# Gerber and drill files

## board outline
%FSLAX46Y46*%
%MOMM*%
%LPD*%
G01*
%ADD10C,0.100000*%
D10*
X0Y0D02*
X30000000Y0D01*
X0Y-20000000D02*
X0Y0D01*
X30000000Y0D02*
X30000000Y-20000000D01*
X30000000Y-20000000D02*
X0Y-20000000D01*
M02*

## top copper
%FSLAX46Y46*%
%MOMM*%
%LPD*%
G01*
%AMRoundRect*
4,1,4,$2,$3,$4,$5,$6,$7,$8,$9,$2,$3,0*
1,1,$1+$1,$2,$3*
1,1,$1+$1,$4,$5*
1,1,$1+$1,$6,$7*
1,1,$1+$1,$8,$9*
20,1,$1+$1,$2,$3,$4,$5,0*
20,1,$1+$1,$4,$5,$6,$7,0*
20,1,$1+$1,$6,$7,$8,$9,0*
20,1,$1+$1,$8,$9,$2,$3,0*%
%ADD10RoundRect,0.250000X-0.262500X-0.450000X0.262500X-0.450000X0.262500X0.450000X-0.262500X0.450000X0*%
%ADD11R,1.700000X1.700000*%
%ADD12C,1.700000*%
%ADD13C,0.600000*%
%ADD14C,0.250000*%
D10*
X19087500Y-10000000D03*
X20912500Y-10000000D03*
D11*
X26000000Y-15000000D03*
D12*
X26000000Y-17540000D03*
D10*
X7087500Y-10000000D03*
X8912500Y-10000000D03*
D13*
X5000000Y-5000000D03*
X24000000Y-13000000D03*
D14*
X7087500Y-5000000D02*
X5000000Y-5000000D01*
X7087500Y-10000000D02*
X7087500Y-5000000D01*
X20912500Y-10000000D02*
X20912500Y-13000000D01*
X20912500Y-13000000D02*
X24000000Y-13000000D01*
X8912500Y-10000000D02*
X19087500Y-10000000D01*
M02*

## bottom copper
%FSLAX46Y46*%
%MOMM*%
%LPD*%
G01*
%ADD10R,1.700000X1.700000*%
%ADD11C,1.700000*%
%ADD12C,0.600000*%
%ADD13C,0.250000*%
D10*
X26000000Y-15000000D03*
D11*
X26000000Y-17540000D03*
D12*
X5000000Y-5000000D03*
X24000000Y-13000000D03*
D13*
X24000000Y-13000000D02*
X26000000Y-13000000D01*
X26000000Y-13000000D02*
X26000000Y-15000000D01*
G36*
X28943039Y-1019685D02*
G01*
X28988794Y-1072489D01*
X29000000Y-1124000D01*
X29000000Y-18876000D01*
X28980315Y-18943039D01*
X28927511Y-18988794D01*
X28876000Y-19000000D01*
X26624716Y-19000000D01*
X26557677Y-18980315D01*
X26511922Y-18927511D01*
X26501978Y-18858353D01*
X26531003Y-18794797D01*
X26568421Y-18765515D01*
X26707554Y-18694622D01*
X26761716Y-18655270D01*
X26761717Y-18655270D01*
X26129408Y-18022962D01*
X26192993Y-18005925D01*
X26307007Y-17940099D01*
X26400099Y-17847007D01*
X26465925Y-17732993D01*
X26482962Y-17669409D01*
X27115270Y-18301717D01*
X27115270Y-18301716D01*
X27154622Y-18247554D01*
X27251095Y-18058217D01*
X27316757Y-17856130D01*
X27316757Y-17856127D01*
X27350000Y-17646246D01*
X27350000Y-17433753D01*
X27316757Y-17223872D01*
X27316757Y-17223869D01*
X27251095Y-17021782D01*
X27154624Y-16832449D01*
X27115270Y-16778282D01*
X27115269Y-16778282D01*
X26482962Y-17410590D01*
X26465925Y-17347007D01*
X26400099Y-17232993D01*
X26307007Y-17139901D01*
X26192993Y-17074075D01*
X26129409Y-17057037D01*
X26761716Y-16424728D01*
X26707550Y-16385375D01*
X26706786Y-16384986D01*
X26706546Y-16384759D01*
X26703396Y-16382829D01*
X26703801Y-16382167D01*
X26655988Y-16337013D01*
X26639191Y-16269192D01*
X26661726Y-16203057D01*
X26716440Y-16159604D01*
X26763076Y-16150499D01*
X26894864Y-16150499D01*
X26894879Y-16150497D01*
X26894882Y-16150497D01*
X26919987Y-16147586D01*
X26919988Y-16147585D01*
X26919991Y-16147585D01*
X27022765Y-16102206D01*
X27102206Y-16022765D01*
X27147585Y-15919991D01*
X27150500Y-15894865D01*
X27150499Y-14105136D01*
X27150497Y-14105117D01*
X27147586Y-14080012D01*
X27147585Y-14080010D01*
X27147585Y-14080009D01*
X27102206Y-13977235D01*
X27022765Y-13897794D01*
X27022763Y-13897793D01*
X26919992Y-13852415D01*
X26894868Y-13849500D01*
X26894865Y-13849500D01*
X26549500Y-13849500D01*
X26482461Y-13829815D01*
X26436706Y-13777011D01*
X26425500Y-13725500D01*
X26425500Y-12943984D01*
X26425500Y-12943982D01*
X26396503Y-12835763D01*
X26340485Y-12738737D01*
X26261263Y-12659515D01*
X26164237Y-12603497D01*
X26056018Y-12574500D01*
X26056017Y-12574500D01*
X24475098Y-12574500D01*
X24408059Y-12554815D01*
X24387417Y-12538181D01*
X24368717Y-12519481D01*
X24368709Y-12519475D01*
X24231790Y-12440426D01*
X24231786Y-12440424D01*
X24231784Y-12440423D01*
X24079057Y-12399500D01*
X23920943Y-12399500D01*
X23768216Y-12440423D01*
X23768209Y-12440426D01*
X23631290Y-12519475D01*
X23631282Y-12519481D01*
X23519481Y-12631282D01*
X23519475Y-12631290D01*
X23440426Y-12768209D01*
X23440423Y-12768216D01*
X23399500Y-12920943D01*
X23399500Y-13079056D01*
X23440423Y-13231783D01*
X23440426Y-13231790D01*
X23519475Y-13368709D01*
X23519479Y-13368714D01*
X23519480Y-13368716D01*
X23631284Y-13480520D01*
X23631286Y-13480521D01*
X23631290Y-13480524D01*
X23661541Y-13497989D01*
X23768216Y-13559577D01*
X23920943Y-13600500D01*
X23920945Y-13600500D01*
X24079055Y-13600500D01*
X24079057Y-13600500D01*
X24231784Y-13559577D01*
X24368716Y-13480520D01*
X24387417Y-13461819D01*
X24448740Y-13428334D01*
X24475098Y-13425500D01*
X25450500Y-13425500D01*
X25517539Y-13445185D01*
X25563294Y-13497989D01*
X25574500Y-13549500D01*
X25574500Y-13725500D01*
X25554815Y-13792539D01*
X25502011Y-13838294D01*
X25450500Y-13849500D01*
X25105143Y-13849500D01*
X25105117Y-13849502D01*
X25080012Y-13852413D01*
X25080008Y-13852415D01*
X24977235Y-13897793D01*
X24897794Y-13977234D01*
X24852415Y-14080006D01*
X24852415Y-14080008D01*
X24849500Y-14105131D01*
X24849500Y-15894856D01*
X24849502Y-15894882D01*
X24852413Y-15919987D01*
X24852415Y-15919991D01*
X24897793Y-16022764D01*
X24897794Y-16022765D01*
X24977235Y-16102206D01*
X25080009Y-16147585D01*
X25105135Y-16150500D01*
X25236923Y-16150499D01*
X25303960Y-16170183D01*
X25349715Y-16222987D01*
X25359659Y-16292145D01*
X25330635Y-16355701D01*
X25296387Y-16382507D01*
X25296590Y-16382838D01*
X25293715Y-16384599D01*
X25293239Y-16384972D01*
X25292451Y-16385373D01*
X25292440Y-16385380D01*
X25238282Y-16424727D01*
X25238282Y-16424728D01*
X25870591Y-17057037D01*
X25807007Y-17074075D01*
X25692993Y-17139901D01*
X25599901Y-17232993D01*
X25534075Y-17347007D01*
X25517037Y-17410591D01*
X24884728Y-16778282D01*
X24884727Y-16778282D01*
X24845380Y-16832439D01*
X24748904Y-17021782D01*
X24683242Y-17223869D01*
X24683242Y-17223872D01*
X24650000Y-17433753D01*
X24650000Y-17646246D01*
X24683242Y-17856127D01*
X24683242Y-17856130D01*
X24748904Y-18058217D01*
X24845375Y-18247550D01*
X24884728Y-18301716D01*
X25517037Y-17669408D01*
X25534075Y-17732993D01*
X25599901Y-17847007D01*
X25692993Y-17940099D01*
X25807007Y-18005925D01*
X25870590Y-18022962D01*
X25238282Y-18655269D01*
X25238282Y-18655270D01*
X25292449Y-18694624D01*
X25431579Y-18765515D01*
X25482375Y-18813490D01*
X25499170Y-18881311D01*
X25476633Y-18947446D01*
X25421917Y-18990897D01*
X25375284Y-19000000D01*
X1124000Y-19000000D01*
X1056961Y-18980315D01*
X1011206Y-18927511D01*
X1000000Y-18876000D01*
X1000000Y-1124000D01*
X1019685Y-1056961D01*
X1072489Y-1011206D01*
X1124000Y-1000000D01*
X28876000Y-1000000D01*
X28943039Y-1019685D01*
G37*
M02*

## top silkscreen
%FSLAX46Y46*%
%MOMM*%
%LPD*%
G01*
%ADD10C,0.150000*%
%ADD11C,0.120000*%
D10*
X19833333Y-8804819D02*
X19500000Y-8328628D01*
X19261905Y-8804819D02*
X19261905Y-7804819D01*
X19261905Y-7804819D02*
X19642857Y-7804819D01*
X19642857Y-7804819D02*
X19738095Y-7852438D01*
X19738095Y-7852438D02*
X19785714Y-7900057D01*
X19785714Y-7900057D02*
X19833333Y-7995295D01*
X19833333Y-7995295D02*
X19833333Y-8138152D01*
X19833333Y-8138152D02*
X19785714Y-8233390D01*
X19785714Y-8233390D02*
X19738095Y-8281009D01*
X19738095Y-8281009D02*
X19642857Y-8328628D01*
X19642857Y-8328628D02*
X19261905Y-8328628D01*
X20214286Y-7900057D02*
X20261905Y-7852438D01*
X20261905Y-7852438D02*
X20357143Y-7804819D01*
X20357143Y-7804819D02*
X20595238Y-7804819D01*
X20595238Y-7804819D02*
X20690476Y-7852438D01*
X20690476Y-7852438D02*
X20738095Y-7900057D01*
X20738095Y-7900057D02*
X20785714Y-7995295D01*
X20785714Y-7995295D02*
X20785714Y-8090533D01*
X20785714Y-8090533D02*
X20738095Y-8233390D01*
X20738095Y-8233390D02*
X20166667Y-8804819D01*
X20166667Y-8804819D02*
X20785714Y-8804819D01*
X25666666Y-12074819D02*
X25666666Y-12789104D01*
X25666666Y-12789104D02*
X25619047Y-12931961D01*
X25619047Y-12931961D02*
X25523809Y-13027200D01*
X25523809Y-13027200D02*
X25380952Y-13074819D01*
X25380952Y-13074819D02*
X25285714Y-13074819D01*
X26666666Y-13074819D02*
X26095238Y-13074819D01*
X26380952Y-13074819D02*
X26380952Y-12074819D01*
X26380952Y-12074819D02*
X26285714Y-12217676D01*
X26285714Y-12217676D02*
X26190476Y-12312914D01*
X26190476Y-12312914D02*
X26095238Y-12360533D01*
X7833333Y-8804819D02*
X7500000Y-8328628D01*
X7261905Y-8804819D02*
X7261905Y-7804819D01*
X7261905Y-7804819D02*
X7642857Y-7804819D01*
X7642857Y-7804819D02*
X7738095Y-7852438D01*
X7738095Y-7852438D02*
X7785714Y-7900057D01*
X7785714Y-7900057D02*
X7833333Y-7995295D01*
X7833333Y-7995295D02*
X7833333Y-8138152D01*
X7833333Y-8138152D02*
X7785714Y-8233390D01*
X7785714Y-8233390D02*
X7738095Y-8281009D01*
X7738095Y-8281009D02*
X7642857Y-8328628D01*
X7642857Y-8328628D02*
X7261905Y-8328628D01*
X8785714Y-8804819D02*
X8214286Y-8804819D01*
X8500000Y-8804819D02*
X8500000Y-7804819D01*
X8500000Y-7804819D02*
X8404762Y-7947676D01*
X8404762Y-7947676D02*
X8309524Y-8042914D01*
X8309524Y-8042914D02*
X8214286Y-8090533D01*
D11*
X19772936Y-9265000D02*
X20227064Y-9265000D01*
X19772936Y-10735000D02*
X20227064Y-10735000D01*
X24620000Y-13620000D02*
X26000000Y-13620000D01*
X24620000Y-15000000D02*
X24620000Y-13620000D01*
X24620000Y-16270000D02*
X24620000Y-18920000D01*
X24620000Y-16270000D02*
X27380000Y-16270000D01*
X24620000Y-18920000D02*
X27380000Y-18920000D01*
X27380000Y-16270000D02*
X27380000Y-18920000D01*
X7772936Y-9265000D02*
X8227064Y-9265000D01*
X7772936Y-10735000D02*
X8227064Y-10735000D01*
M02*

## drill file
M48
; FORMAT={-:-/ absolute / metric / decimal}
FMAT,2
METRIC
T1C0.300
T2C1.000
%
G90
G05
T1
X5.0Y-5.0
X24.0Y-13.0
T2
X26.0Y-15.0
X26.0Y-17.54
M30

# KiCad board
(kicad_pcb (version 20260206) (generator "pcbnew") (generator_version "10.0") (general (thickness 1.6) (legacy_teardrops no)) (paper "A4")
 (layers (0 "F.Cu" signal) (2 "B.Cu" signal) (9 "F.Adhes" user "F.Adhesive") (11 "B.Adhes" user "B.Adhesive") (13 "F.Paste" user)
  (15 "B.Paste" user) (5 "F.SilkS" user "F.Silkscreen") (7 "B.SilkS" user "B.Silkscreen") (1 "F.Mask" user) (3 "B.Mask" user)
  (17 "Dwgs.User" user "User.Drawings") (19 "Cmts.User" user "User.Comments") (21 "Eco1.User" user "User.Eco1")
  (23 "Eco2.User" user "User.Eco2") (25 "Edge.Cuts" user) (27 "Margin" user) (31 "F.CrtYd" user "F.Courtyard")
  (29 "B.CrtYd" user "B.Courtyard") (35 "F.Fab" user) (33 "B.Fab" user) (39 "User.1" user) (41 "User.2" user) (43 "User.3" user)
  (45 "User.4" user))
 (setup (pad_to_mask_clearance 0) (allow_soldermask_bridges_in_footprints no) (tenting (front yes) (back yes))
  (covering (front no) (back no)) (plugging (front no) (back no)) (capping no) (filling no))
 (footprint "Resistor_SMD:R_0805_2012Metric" (layer "F.Cu") (at 20 10)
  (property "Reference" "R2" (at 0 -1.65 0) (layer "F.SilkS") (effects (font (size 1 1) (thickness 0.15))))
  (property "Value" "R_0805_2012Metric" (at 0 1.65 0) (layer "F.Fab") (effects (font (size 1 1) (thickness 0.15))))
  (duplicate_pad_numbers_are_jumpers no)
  (fp_line (start -0.227064 -0.735) (end 0.227064 -0.735) (stroke (width 0.12) (type solid)) (layer "F.SilkS"))
  (fp_line (start -0.227064 0.735) (end 0.227064 0.735) (stroke (width 0.12) (type solid)) (layer "F.SilkS"))
  (pad "1" smd roundrect (at -0.9125 0) (size 1.025 1.4) (layers "F.Cu" "F.Mask" "F.Paste") (roundrect_rratio 0.243902) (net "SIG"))
  (pad "2" smd roundrect (at 0.9125 0) (size 1.025 1.4) (layers "F.Cu" "F.Mask" "F.Paste") (roundrect_rratio 0.243902) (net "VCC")))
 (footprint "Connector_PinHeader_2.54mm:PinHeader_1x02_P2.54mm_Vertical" (layer "F.Cu") (at 26 15)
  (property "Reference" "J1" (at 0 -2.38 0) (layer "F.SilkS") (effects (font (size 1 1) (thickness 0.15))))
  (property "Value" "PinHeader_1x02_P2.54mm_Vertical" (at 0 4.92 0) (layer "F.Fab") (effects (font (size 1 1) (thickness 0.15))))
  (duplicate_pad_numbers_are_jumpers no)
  (fp_line (start -1.38 -1.38) (end 0 -1.38) (stroke (width 0.12) (type solid)) (layer "F.SilkS"))
  (fp_line (start -1.38 0) (end -1.38 -1.38) (stroke (width 0.12) (type solid)) (layer "F.SilkS"))
  (fp_line (start -1.38 1.27) (end -1.38 3.92) (stroke (width 0.12) (type solid)) (layer "F.SilkS"))
  (fp_line (start -1.38 1.27) (end 1.38 1.27) (stroke (width 0.12) (type solid)) (layer "F.SilkS"))
  (fp_line (start -1.38 3.92) (end 1.38 3.92) (stroke (width 0.12) (type solid)) (layer "F.SilkS"))
  (fp_line (start 1.38 1.27) (end 1.38 3.92) (stroke (width 0.12) (type solid)) (layer "F.SilkS"))
  (pad "1" thru_hole rect (at 0 0) (size 1.7 1.7) (drill 1) (layers "*.Cu" "*.Mask") (remove_unused_layers no) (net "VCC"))
  (pad "2" thru_hole circle (at 0 2.54) (size 1.7 1.7) (drill 1) (layers "*.Cu" "*.Mask") (remove_unused_layers no) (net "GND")))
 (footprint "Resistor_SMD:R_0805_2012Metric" (layer "F.Cu") (at 8 10)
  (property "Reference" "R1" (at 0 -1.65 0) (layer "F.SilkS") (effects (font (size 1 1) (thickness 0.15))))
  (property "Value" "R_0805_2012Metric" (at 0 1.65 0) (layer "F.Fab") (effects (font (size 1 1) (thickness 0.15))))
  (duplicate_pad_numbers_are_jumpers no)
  (fp_line (start -0.227064 -0.735) (end 0.227064 -0.735) (stroke (width 0.12) (type solid)) (layer "F.SilkS"))
  (fp_line (start -0.227064 0.735) (end 0.227064 0.735) (stroke (width 0.12) (type solid)) (layer "F.SilkS"))
  (pad "1" smd roundrect (at -0.9125 0) (size 1.025 1.4) (layers "F.Cu" "F.Mask" "F.Paste") (roundrect_rratio 0.243902) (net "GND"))
  (pad "2" smd roundrect (at 0.9125 0) (size 1.025 1.4) (layers "F.Cu" "F.Mask" "F.Paste") (roundrect_rratio 0.243902) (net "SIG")))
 (gr_line (start 0 0) (end 30 0) (stroke (width 0.1) (type default)) (layer "Edge.Cuts"))
 (gr_line (start 0 20) (end 0 0) (stroke (width 0.1) (type default)) (layer "Edge.Cuts"))
 (gr_line (start 30 0) (end 30 20) (stroke (width 0.1) (type default)) (layer "Edge.Cuts"))
 (gr_line (start 30 20) (end 0 20) (stroke (width 0.1) (type default)) (layer "Edge.Cuts"))
 (segment (start 7.0875 5) (end 5 5) (width 0.25) (layer "F.Cu") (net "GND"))
 (segment (start 7.0875 10) (end 7.0875 5) (width 0.25) (layer "F.Cu") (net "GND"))
 (via (at 5 5) (size 0.6) (drill 0.3) (layers "F.Cu" "B.Cu") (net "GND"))
 (segment (start 20.9125 10) (end 20.9125 13) (width 0.25) (layer "F.Cu") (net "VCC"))
 (segment (start 20.9125 13) (end 24 13) (width 0.25) (layer "F.Cu") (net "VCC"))
 (via (at 24 13) (size 0.6) (drill 0.3) (layers "F.Cu" "B.Cu") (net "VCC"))
 (segment (start 24 13) (end 26 13) (width 0.25) (layer "B.Cu") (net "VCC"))
 (segment (start 26 13) (end 26 15) (width 0.25) (layer "B.Cu") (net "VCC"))
 (segment (start 8.9125 10) (end 19.0875 10) (width 0.25) (layer "F.Cu") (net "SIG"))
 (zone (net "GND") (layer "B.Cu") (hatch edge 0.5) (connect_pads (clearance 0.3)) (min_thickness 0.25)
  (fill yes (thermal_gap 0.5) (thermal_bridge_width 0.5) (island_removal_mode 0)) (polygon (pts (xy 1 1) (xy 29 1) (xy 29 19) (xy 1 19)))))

